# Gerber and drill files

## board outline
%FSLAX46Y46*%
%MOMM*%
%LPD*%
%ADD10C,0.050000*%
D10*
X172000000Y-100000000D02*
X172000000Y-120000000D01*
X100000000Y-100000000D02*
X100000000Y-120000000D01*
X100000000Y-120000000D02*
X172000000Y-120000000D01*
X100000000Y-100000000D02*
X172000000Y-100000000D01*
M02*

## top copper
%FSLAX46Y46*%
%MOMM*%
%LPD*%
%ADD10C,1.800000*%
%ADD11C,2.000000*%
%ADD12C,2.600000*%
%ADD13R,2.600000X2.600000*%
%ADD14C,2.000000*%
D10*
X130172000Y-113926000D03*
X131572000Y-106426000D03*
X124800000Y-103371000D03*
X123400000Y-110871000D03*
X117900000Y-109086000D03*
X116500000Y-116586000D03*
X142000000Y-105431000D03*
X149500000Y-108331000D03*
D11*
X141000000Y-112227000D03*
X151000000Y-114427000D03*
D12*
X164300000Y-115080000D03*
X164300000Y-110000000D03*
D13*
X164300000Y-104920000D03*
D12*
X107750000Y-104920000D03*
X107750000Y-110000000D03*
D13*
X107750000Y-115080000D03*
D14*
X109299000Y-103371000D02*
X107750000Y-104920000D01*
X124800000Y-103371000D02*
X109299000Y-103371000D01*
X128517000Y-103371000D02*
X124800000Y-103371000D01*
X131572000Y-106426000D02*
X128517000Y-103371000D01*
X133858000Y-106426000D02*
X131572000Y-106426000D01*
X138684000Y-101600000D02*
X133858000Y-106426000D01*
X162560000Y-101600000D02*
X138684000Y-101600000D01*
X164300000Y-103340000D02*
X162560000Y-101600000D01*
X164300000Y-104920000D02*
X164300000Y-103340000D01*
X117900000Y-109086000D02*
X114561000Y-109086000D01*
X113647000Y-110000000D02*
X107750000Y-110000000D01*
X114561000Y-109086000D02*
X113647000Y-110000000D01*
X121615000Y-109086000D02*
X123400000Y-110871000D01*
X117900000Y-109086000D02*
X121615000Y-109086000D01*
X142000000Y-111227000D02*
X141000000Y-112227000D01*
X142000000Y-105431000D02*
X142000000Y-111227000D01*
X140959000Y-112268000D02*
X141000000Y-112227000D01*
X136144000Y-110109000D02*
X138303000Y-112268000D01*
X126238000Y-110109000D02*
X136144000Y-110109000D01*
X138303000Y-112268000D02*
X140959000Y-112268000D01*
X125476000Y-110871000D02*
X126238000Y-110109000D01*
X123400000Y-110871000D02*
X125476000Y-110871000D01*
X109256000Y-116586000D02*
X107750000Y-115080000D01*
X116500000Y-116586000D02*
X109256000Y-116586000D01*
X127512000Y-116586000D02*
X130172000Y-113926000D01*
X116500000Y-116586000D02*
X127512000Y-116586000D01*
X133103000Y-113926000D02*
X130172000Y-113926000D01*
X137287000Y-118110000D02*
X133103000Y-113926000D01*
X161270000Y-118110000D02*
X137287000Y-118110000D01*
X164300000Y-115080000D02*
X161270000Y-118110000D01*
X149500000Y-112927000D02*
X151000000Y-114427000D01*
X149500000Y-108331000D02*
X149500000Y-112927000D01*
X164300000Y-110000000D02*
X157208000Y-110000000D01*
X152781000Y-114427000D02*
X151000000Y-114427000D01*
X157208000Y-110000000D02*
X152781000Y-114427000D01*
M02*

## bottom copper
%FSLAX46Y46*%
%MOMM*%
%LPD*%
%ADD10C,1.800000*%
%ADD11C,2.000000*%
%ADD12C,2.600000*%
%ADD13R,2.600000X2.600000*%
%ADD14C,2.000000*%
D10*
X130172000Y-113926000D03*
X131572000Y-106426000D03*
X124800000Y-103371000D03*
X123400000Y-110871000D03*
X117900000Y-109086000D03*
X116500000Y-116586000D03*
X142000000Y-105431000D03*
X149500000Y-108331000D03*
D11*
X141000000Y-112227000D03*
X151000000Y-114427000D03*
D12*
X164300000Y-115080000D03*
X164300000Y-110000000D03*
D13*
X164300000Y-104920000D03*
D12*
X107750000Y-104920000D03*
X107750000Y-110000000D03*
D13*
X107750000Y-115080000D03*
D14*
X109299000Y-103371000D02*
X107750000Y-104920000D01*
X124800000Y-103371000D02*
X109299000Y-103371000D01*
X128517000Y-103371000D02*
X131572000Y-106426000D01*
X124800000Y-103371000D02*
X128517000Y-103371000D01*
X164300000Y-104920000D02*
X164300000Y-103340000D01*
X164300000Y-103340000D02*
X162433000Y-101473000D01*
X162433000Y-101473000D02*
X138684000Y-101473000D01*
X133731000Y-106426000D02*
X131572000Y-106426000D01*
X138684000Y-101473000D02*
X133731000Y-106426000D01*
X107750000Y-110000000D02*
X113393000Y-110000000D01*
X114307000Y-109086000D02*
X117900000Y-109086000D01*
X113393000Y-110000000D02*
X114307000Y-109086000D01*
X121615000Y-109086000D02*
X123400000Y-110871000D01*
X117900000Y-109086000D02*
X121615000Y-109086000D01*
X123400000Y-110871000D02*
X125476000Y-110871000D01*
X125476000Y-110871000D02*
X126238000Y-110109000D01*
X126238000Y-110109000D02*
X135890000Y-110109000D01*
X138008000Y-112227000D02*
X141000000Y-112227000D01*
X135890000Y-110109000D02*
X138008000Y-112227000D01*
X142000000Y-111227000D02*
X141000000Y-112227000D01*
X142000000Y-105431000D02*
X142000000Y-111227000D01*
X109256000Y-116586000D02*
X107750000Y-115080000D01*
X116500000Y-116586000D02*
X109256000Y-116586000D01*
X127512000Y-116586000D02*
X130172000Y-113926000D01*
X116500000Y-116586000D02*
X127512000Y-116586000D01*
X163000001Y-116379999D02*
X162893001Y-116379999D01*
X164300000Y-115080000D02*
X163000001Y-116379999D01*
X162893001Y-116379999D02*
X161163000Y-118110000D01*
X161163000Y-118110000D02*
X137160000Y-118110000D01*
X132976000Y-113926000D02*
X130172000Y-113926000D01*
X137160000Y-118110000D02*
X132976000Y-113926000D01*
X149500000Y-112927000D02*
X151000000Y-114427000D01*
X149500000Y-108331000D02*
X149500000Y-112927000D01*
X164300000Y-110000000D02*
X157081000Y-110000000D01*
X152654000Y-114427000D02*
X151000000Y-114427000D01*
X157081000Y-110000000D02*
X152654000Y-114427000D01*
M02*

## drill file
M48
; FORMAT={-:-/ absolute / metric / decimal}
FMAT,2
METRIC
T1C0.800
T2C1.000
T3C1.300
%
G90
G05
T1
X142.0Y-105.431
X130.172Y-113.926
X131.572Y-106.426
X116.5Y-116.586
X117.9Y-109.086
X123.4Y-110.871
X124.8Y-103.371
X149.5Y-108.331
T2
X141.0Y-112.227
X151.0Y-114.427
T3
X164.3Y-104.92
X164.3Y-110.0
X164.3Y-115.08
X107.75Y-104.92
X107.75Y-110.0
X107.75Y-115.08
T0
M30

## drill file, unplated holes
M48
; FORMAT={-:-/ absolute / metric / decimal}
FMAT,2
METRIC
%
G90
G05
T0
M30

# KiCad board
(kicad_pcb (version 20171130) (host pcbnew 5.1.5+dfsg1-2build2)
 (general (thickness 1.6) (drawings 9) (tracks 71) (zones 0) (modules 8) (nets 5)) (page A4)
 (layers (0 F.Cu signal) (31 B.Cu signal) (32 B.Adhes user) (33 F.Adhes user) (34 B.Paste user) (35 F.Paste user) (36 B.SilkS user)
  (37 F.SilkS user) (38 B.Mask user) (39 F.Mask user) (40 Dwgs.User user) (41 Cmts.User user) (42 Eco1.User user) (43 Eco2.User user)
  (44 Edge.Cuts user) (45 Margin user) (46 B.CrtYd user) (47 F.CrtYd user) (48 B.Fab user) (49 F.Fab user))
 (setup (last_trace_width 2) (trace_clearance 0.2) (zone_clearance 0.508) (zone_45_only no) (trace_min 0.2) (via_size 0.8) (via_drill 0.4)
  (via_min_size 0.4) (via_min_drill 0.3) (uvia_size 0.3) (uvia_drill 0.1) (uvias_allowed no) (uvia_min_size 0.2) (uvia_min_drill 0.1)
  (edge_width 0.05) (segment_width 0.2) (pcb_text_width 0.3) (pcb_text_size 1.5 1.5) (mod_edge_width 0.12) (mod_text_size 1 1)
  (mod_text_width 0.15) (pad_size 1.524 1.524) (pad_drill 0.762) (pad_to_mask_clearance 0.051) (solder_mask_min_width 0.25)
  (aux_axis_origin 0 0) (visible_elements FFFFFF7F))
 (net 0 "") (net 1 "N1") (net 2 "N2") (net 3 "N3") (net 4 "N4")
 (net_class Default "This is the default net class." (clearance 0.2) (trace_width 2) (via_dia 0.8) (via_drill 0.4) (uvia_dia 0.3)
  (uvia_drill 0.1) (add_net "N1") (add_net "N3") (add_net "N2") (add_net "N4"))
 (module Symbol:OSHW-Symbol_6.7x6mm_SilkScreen (layer F.Cu) (at 117.221 103.251 180)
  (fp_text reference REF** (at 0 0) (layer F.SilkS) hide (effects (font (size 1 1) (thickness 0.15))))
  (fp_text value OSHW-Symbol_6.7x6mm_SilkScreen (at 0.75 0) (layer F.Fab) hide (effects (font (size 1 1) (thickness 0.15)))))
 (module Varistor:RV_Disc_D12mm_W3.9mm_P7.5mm (layer F.Cu) (at 131.572 106.426 270)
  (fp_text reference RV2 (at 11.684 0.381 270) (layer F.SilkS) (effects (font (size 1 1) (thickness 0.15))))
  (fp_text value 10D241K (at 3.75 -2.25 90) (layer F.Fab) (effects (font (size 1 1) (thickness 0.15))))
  (pad 2 thru_hole circle (at 7.5 1.4 270) (size 1.8 1.8) (drill 0.8) (layers *.Cu *.Mask) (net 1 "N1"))
  (pad 1 thru_hole circle (at 0 0 270) (size 1.8 1.8) (drill 0.8) (layers *.Cu *.Mask) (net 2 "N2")))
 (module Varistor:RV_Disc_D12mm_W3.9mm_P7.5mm (layer F.Cu) (at 123.4 110.871 90)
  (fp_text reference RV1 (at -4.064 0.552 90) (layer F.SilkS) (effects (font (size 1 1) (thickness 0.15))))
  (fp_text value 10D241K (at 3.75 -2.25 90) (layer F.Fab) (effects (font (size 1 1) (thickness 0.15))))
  (pad 2 thru_hole circle (at 7.5 1.4 90) (size 1.8 1.8) (drill 0.8) (layers *.Cu *.Mask) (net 2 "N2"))
  (pad 1 thru_hole circle (at 0 0 90) (size 1.8 1.8) (drill 0.8) (layers *.Cu *.Mask) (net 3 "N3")))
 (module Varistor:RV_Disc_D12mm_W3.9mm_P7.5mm (layer F.Cu) (at 116.5 116.586 90)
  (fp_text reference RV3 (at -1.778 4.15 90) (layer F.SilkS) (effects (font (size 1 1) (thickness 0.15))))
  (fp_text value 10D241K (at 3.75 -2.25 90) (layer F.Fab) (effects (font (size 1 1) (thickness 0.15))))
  (pad 2 thru_hole circle (at 7.5 1.4 90) (size 1.8 1.8) (drill 0.8) (layers *.Cu *.Mask) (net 3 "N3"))
  (pad 1 thru_hole circle (at 0 0 90) (size 1.8 1.8) (drill 0.8) (layers *.Cu *.Mask) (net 1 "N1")))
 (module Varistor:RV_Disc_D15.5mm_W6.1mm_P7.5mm (layer F.Cu) (at 149.5 108.331 180)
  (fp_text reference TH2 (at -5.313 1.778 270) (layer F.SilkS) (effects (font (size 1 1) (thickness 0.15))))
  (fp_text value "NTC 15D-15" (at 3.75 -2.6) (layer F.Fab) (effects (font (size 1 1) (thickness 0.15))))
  (pad 2 thru_hole circle (at 7.5 2.9 180) (size 1.8 1.8) (drill 0.8) (layers *.Cu *.Mask) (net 3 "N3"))
  (pad 1 thru_hole circle (at 0 0 180) (size 1.8 1.8) (drill 0.8) (layers *.Cu *.Mask) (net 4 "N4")))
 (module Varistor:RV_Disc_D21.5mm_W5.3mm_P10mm (layer F.Cu) (at 151 114.427 180)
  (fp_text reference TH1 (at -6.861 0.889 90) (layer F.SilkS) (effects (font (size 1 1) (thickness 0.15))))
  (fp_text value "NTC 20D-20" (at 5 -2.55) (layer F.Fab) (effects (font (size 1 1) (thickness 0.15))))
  (pad 2 thru_hole circle (at 10 2.2 180) (size 2 2) (drill 1) (layers *.Cu *.Mask) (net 3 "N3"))
  (pad 1 thru_hole circle (at 0 0 180) (size 2 2) (drill 1) (layers *.Cu *.Mask) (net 4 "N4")))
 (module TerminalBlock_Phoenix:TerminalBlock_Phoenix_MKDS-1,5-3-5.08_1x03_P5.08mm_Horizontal (layer F.Cu) (at 164.3 104.92 270)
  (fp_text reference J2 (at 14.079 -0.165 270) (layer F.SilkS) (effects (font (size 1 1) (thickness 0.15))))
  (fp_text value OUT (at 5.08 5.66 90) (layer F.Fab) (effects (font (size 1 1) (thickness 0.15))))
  (pad 3 thru_hole circle (at 10.16 0 270) (size 2.6 2.6) (drill 1.3) (layers *.Cu *.Mask) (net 1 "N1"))
  (pad 2 thru_hole circle (at 5.08 0 270) (size 2.6 2.6) (drill 1.3) (layers *.Cu *.Mask) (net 4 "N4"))
  (pad 1 thru_hole rect (at 0 0 270) (size 2.6 2.6) (drill 1.3) (layers *.Cu *.Mask) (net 2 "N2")))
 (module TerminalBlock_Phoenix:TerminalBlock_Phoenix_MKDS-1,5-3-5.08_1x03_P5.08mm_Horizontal (layer F.Cu) (at 107.75 115.08 90)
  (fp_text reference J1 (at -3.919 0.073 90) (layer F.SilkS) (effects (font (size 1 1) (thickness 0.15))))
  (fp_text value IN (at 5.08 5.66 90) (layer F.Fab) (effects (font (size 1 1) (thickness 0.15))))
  (pad 3 thru_hole circle (at 10.16 0 90) (size 2.6 2.6) (drill 1.3) (layers *.Cu *.Mask) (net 2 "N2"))
  (pad 2 thru_hole circle (at 5.08 0 90) (size 2.6 2.6) (drill 1.3) (layers *.Cu *.Mask) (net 3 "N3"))
  (pad 1 thru_hole rect (at 0 0 90) (size 2.6 2.6) (drill 1.3) (layers *.Cu *.Mask) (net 1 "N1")))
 (gr_line (start 172 100) (end 172 120) (layer Edge.Cuts) (width 0.05))
 (gr_line (start 100 100) (end 100 120) (layer Edge.Cuts) (width 0.05))
 (gr_line (start 100 120) (end 172 120) (layer Edge.Cuts) (width 0.05))
 (gr_line (start 100 100) (end 172 100) (layer Edge.Cuts) (width 0.05))
 (segment (start 109.299 103.371) (end 107.75 104.92) (width 2) (layer F.Cu) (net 2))
 (segment (start 124.8 103.371) (end 109.299 103.371) (width 2) (layer F.Cu) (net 2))
 (segment (start 128.517 103.371) (end 124.8 103.371) (width 2) (layer F.Cu) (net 2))
 (segment (start 131.572 106.426) (end 128.517 103.371) (width 2) (layer F.Cu) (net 2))
 (segment (start 133.858 106.426) (end 131.572 106.426) (width 2) (layer F.Cu) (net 2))
 (segment (start 138.684 101.6) (end 133.858 106.426) (width 2) (layer F.Cu) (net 2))
 (segment (start 162.56 101.6) (end 138.684 101.6) (width 2) (layer F.Cu) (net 2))
 (segment (start 164.3 103.34) (end 162.56 101.6) (width 2) (layer F.Cu) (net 2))
 (segment (start 164.3 104.92) (end 164.3 103.34) (width 2) (layer F.Cu) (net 2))
 (segment (start 109.299 103.371) (end 107.75 104.92) (width 2) (layer B.Cu) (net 2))
 (segment (start 124.8 103.371) (end 109.299 103.371) (width 2) (layer B.Cu) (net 2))
 (segment (start 128.517 103.371) (end 131.572 106.426) (width 2) (layer B.Cu) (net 2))
 (segment (start 124.8 103.371) (end 128.517 103.371) (width 2) (layer B.Cu) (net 2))
 (segment (start 164.3 104.92) (end 164.3 103.34) (width 2) (layer B.Cu) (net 2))
 (segment (start 164.3 103.34) (end 162.433 101.473) (width 2) (layer B.Cu) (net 2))
 (segment (start 162.433 101.473) (end 138.684 101.473) (width 2) (layer B.Cu) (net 2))
 (segment (start 133.731 106.426) (end 131.572 106.426) (width 2) (layer B.Cu) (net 2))
 (segment (start 138.684 101.473) (end 133.731 106.426) (width 2) (layer B.Cu) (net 2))
 (segment (start 117.9 109.086) (end 114.561 109.086) (width 2) (layer F.Cu) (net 3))
 (segment (start 113.647 110) (end 107.75 110) (width 2) (layer F.Cu) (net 3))
 (segment (start 114.561 109.086) (end 113.647 110) (width 2) (layer F.Cu) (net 3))
 (segment (start 121.615 109.086) (end 123.4 110.871) (width 2) (layer F.Cu) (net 3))
 (segment (start 117.9 109.086) (end 121.615 109.086) (width 2) (layer F.Cu) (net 3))
 (segment (start 142 111.227) (end 141 112.227) (width 2) (layer F.Cu) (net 3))
 (segment (start 142 105.431) (end 142 111.227) (width 2) (layer F.Cu) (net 3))
 (segment (start 140.959 112.268) (end 141 112.227) (width 2) (layer F.Cu) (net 3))
 (segment (start 136.144 110.109) (end 138.303 112.268) (width 2) (layer F.Cu) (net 3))
 (segment (start 126.238 110.109) (end 136.144 110.109) (width 2) (layer F.Cu) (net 3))
 (segment (start 138.303 112.268) (end 140.959 112.268) (width 2) (layer F.Cu) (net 3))
 (segment (start 125.476 110.871) (end 126.238 110.109) (width 2) (layer F.Cu) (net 3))
 (segment (start 123.4 110.871) (end 125.476 110.871) (width 2) (layer F.Cu) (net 3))
 (segment (start 107.75 110) (end 113.393 110) (width 2) (layer B.Cu) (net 3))
 (segment (start 114.307 109.086) (end 117.9 109.086) (width 2) (layer B.Cu) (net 3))
 (segment (start 113.393 110) (end 114.307 109.086) (width 2) (layer B.Cu) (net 3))
 (segment (start 121.615 109.086) (end 123.4 110.871) (width 2) (layer B.Cu) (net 3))
 (segment (start 117.9 109.086) (end 121.615 109.086) (width 2) (layer B.Cu) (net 3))
 (segment (start 123.4 110.871) (end 125.476 110.871) (width 2) (layer B.Cu) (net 3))
 (segment (start 125.476 110.871) (end 126.238 110.109) (width 2) (layer B.Cu) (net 3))
 (segment (start 126.238 110.109) (end 135.89 110.109) (width 2) (layer B.Cu) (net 3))
 (segment (start 138.008 112.227) (end 141 112.227) (width 2) (layer B.Cu) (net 3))
 (segment (start 135.89 110.109) (end 138.008 112.227) (width 2) (layer B.Cu) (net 3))
 (segment (start 142 111.227) (end 141 112.227) (width 2) (layer B.Cu) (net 3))
 (segment (start 142 105.431) (end 142 111.227) (width 2) (layer B.Cu) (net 3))
 (segment (start 109.256 116.586) (end 107.75 115.08) (width 2) (layer F.Cu) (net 1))
 (segment (start 116.5 116.586) (end 109.256 116.586) (width 2) (layer F.Cu) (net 1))
 (segment (start 127.512 116.586) (end 130.172 113.926) (width 2) (layer F.Cu) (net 1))
 (segment (start 116.5 116.586) (end 127.512 116.586) (width 2) (layer F.Cu) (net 1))
 (segment (start 133.103 113.926) (end 130.172 113.926) (width 2) (layer F.Cu) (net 1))
 (segment (start 137.287 118.11) (end 133.103 113.926) (width 2) (layer F.Cu) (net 1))
 (segment (start 161.27 118.11) (end 137.287 118.11) (width 2) (layer F.Cu) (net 1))
 (segment (start 164.3 115.08) (end 161.27 118.11) (width 2) (layer F.Cu) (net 1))
 (segment (start 109.256 116.586) (end 107.75 115.08) (width 2) (layer B.Cu) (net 1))
 (segment (start 116.5 116.586) (end 109.256 116.586) (width 2) (layer B.Cu) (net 1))
 (segment (start 127.512 116.586) (end 130.172 113.926) (width 2) (layer B.Cu) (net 1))
 (segment (start 116.5 116.586) (end 127.512 116.586) (width 2) (layer B.Cu) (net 1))
 (segment (start 163.000001 116.379999) (end 162.893001 116.379999) (width 2) (layer B.Cu) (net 1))
 (segment (start 164.3 115.08) (end 163.000001 116.379999) (width 2) (layer B.Cu) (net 1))
 (segment (start 162.893001 116.379999) (end 161.163 118.11) (width 2) (layer B.Cu) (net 1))
 (segment (start 161.163 118.11) (end 137.16 118.11) (width 2) (layer B.Cu) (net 1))
 (segment (start 132.976 113.926) (end 130.172 113.926) (width 2) (layer B.Cu) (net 1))
 (segment (start 137.16 118.11) (end 132.976 113.926) (width 2) (layer B.Cu) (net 1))
 (segment (start 149.5 112.927) (end 151 114.427) (width 2) (layer F.Cu) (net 4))
 (segment (start 149.5 108.331) (end 149.5 112.927) (width 2) (layer F.Cu) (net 4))
 (segment (start 164.3 110) (end 157.208 110) (width 2) (layer F.Cu) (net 4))
 (segment (start 152.781 114.427) (end 151 114.427) (width 2) (layer F.Cu) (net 4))
 (segment (start 157.208 110) (end 152.781 114.427) (width 2) (layer F.Cu) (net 4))
 (segment (start 149.5 112.927) (end 151 114.427) (width 2) (layer B.Cu) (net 4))
 (segment (start 149.5 108.331) (end 149.5 112.927) (width 2) (layer B.Cu) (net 4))
 (segment (start 164.3 110) (end 157.081 110) (width 2) (layer B.Cu) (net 4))
 (segment (start 152.654 114.427) (end 151 114.427) (width 2) (layer B.Cu) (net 4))
 (segment (start 157.081 110) (end 152.654 114.427) (width 2) (layer B.Cu) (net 4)))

